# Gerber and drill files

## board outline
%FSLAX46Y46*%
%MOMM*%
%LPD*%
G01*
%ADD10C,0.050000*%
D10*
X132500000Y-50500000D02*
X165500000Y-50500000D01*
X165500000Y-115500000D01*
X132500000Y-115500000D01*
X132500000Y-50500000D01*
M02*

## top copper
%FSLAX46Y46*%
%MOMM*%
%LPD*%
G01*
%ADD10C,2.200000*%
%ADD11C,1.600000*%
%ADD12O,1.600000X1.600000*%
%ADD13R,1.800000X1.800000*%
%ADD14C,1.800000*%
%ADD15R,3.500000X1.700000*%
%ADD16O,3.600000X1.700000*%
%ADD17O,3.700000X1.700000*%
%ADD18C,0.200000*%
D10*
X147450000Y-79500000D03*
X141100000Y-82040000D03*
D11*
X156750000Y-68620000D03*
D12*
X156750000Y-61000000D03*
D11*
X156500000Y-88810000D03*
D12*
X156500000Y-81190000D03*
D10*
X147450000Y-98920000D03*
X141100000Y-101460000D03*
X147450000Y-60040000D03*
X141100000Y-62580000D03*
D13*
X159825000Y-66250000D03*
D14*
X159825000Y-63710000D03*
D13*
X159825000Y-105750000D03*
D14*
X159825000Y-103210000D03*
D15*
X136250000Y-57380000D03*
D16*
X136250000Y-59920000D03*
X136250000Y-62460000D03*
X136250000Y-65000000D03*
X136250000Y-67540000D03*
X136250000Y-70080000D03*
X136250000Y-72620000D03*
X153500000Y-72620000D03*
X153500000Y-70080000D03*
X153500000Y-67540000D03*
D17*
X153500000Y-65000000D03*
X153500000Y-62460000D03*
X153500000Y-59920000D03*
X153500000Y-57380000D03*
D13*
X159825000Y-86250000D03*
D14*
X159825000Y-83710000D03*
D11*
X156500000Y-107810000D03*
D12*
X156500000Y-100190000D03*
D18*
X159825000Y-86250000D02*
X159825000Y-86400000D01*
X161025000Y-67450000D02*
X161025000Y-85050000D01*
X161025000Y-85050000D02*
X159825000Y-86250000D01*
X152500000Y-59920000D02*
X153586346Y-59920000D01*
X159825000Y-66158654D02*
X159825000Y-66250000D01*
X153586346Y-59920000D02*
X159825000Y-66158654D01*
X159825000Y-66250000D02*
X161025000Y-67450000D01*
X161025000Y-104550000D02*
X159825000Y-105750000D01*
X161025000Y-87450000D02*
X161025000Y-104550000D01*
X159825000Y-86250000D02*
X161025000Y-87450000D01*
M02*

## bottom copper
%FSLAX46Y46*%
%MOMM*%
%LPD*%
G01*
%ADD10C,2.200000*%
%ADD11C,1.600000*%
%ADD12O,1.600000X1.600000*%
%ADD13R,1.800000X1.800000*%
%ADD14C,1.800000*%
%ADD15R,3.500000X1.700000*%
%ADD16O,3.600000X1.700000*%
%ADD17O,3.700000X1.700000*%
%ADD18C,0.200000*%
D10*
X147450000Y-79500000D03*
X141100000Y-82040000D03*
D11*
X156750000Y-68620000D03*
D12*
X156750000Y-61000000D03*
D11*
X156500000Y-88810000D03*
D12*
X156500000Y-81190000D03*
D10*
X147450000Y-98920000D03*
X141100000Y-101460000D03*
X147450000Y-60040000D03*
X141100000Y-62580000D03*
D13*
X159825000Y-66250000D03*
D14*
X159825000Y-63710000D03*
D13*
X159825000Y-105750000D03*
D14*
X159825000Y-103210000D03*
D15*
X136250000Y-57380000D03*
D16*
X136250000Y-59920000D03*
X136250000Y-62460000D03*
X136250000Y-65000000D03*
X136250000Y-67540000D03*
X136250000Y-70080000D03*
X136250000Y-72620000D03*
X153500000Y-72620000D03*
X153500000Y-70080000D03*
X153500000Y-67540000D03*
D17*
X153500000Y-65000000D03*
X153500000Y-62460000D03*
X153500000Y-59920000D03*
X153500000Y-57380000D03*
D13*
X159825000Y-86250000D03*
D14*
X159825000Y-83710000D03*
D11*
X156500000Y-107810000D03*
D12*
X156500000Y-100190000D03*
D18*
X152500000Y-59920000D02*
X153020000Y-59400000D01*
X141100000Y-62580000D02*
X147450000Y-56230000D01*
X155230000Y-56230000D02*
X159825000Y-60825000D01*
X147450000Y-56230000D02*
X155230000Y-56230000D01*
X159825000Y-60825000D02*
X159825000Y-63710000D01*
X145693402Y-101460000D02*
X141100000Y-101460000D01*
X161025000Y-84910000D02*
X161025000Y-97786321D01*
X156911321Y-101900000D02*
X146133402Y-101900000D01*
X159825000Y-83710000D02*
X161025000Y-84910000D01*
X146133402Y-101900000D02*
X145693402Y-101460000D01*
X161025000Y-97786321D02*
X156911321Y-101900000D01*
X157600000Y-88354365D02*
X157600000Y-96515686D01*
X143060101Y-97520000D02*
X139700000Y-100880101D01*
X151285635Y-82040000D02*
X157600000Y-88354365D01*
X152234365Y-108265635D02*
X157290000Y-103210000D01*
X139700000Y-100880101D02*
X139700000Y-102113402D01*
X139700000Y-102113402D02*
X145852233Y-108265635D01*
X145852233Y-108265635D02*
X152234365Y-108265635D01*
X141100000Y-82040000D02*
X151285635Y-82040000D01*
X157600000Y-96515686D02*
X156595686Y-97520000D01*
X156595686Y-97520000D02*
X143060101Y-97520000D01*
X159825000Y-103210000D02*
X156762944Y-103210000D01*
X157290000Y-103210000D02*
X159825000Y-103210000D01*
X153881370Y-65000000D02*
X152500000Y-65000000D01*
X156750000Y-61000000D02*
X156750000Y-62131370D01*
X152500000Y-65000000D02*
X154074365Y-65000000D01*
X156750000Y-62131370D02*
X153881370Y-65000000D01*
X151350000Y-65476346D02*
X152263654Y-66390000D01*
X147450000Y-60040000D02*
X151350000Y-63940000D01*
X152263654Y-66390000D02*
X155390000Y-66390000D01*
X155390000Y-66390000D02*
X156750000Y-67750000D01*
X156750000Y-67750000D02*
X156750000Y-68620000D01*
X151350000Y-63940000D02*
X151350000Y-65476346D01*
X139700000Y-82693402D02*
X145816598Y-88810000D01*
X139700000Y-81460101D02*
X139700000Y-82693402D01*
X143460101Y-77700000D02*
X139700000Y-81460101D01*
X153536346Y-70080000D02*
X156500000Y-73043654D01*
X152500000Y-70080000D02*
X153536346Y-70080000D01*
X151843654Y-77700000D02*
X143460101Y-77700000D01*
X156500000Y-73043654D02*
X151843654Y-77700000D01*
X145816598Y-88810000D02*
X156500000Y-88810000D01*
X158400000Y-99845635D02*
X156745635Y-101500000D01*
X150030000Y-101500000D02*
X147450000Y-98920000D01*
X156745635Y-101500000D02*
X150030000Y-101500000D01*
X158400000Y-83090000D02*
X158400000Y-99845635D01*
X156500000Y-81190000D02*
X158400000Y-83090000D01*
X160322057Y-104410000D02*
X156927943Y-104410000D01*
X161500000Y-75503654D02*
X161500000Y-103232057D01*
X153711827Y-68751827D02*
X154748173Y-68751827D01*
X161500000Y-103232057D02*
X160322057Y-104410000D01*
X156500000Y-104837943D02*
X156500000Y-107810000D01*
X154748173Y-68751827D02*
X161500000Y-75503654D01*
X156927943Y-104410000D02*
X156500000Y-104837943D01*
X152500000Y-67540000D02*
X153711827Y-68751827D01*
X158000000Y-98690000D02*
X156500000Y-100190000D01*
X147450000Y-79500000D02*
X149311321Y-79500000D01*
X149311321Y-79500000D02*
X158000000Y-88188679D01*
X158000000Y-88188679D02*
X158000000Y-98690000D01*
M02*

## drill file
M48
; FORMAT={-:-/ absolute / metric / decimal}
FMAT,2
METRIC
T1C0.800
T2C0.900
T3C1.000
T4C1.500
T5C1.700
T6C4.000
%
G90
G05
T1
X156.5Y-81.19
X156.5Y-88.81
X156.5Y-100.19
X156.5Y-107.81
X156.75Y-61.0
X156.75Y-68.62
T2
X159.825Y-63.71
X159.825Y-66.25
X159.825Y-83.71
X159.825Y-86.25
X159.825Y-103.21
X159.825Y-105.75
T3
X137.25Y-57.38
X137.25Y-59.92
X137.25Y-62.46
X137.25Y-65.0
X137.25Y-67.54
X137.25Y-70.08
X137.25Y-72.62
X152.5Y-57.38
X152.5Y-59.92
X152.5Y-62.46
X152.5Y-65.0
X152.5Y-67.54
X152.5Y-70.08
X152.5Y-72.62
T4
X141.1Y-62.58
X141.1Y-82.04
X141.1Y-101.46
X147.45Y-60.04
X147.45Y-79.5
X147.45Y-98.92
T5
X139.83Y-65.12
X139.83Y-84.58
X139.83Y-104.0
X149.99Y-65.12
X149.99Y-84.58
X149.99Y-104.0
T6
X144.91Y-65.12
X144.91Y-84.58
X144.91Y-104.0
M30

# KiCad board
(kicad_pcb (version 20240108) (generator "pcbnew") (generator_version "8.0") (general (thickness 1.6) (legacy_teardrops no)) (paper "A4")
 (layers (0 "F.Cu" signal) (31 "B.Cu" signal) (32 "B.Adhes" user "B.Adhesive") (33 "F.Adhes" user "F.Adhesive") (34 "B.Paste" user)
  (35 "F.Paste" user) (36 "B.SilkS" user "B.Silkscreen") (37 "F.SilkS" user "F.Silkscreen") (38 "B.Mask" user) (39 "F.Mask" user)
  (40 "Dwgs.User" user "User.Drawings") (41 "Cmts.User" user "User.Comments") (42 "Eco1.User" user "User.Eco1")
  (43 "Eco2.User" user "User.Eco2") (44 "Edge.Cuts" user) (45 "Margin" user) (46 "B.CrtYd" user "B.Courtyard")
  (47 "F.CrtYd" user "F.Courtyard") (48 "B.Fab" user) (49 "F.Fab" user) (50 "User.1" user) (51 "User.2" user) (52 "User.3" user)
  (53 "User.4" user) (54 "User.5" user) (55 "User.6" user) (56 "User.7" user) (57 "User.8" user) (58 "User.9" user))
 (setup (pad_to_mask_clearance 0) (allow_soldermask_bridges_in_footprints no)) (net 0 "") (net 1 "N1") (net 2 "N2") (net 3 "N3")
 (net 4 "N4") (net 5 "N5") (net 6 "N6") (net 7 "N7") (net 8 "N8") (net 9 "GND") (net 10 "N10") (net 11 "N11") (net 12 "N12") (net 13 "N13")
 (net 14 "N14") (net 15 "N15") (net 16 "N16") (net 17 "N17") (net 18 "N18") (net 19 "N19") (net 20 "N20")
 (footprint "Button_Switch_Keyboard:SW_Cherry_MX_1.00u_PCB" (layer "F.Cu") (at 147.45 79.5)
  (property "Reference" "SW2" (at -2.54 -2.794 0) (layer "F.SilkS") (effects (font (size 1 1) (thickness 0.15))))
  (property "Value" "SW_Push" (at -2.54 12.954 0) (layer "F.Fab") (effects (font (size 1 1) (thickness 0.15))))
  (pad "" np_thru_hole circle (at -7.62 5.08) (size 1.7 1.7) (drill 1.7) (layers "*.Cu" "*.Mask"))
  (pad "" np_thru_hole circle (at -2.54 5.08) (size 4 4) (drill 4) (layers "*.Cu" "*.Mask"))
  (pad "" np_thru_hole circle (at 2.54 5.08) (size 1.7 1.7) (drill 1.7) (layers "*.Cu" "*.Mask"))
  (pad "1" thru_hole circle (at 0 0) (size 2.2 2.2) (drill 1.5) (layers "*.Cu" "*.Mask") (remove_unused_layers no) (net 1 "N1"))
  (pad "2" thru_hole circle (at -6.35 2.54) (size 2.2 2.2) (drill 1.5) (layers "*.Cu" "*.Mask") (remove_unused_layers no) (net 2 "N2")))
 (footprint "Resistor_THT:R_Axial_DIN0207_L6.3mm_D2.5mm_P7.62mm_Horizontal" (layer "F.Cu") (at 156.75 68.62 90)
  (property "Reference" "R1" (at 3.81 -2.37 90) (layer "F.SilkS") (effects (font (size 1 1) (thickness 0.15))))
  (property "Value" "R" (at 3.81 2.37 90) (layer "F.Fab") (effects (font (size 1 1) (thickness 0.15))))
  (pad "1" thru_hole circle (at 0 0 90) (size 1.6 1.6) (drill 0.8) (layers "*.Cu" "*.Mask") (remove_unused_layers no) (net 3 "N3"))
  (pad "2" thru_hole oval (at 7.62 0 90) (size 1.6 1.6) (drill 0.8) (layers "*.Cu" "*.Mask") (remove_unused_layers no) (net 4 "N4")))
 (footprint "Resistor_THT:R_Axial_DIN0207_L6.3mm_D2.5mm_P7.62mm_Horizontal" (layer "F.Cu") (at 156.5 88.81 90)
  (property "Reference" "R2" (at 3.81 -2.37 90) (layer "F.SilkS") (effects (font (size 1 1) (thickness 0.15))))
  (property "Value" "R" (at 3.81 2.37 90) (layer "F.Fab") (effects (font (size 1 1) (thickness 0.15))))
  (pad "1" thru_hole circle (at 0 0 90) (size 1.6 1.6) (drill 0.8) (layers "*.Cu" "*.Mask") (remove_unused_layers no) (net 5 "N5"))
  (pad "2" thru_hole oval (at 7.62 0 90) (size 1.6 1.6) (drill 0.8) (layers "*.Cu" "*.Mask") (remove_unused_layers no) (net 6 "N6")))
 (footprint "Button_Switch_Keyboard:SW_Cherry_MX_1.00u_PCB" (layer "F.Cu") (at 147.45 98.92)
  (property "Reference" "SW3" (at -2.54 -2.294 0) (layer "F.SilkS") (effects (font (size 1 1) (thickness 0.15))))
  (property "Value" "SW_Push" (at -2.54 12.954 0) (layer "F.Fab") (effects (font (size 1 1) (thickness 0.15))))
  (pad "" np_thru_hole circle (at -7.62 5.08) (size 1.7 1.7) (drill 1.7) (layers "*.Cu" "*.Mask"))
  (pad "" np_thru_hole circle (at -2.54 5.08) (size 4 4) (drill 4) (layers "*.Cu" "*.Mask"))
  (pad "" np_thru_hole circle (at 2.54 5.08) (size 1.7 1.7) (drill 1.7) (layers "*.Cu" "*.Mask"))
  (pad "1" thru_hole circle (at 0 0) (size 2.2 2.2) (drill 1.5) (layers "*.Cu" "*.Mask") (remove_unused_layers no) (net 6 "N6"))
  (pad "2" thru_hole circle (at -6.35 2.54) (size 2.2 2.2) (drill 1.5) (layers "*.Cu" "*.Mask") (remove_unused_layers no) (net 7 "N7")))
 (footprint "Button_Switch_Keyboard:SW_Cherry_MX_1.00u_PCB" (layer "F.Cu") (at 147.45 60.04)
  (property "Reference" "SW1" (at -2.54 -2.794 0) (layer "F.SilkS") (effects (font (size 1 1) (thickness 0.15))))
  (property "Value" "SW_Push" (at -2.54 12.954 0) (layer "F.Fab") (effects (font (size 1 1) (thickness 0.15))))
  (pad "" np_thru_hole circle (at -7.62 5.08) (size 1.7 1.7) (drill 1.7) (layers "*.Cu" "*.Mask"))
  (pad "" np_thru_hole circle (at -2.54 5.08) (size 4 4) (drill 4) (layers "*.Cu" "*.Mask"))
  (pad "" np_thru_hole circle (at 2.54 5.08) (size 1.7 1.7) (drill 1.7) (layers "*.Cu" "*.Mask"))
  (pad "1" thru_hole circle (at 0 0) (size 2.2 2.2) (drill 1.5) (layers "*.Cu" "*.Mask") (remove_unused_layers no) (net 3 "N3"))
  (pad "2" thru_hole circle (at -6.35 2.54) (size 2.2 2.2) (drill 1.5) (layers "*.Cu" "*.Mask") (remove_unused_layers no) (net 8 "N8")))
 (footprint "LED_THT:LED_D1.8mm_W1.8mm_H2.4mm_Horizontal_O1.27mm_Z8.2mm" (layer "F.Cu") (at 159.825 66.25 90)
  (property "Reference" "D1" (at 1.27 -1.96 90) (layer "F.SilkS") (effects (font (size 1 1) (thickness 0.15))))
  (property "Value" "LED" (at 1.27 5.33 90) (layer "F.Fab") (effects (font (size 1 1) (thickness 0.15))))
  (pad "1" thru_hole rect (at 0 0 90) (size 1.8 1.8) (drill 0.9) (layers "*.Cu" "*.Mask") (remove_unused_layers no) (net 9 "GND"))
  (pad "2" thru_hole circle (at 2.54 0 90) (size 1.8 1.8) (drill 0.9) (layers "*.Cu" "*.Mask") (remove_unused_layers no) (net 8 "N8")))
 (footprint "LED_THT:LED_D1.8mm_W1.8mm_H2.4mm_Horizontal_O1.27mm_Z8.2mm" (layer "F.Cu") (at 159.825 105.75 90)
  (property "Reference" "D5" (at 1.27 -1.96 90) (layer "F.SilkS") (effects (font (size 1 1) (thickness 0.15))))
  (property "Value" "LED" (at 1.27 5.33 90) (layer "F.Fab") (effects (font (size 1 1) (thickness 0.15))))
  (pad "1" thru_hole rect (at 0 0 90) (size 1.8 1.8) (drill 0.9) (layers "*.Cu" "*.Mask") (remove_unused_layers no) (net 9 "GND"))
  (pad "2" thru_hole circle (at 2.54 0 90) (size 1.8 1.8) (drill 0.9) (layers "*.Cu" "*.Mask") (remove_unused_layers no) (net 2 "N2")))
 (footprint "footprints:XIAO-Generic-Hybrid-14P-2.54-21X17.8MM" (layer "F.Cu") (at 144.875 65)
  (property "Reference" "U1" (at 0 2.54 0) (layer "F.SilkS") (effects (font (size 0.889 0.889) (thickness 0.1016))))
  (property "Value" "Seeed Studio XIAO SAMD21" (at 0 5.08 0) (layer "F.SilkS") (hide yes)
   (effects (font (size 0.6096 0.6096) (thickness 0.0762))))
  (pad "1" thru_hole rect (at -7.625 -7.62) (size 3.5 1.7) (drill 1 (offset -1 0)) (layers "*.Cu" "*.Mask") (remove_unused_layers no)
   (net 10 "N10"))
  (pad "2" thru_hole oval (at -7.625 -5.08) (size 3.6 1.7) (drill 1 (offset -1 0)) (layers "*.Cu" "*.Mask") (remove_unused_layers no)
   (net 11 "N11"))
  (pad "3" thru_hole oval (at -7.625 -2.54) (size 3.6 1.7) (drill 1 (offset -1 0)) (layers "*.Cu" "*.Mask") (remove_unused_layers no)
   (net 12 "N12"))
  (pad "4" thru_hole oval (at -7.625 0) (size 3.6 1.7) (drill 1 (offset -1 0)) (layers "*.Cu" "*.Mask") (remove_unused_layers no)
   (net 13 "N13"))
  (pad "5" thru_hole oval (at -7.625 2.54) (size 3.6 1.7) (drill 1 (offset -1 0)) (layers "*.Cu" "*.Mask") (remove_unused_layers no)
   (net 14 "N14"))
  (pad "6" thru_hole oval (at -7.625 5.08 180) (size 3.6 1.7) (drill 1 (offset 1 0)) (layers "*.Cu" "*.Mask") (remove_unused_layers no)
   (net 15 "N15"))
  (pad "7" thru_hole oval (at -7.625 7.62) (size 3.6 1.7) (drill 1 (offset -1 0)) (layers "*.Cu" "*.Mask") (remove_unused_layers no)
   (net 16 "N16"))
  (pad "8" thru_hole oval (at 7.625 7.62) (size 3.6 1.7) (drill 1 (offset 1 0)) (layers "*.Cu" "*.Mask") (remove_unused_layers no)
   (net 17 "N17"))
  (pad "9" thru_hole oval (at 7.625 5.08) (size 3.6 1.7) (drill 1 (offset 1 0)) (layers "*.Cu" "*.Mask") (remove_unused_layers no)
   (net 5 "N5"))
  (pad "10" thru_hole oval (at 7.625 2.54) (size 3.6 1.7) (drill 1 (offset 1 0)) (layers "*.Cu" "*.Mask") (remove_unused_layers no)
   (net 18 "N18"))
  (pad "11" thru_hole oval (at 7.625 0) (size 3.7 1.7) (drill 1 (offset 1 0)) (layers "*.Cu" "*.Mask") (remove_unused_layers no)
   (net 4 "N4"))
  (pad "12" thru_hole oval (at 7.625 -2.54) (size 3.7 1.7) (drill 1 (offset 1 0)) (layers "*.Cu" "*.Mask") (remove_unused_layers no)
   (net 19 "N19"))
  (pad "13" thru_hole oval (at 7.625 -5.08) (size 3.7 1.7) (drill 1 (offset 1 0)) (layers "*.Cu" "*.Mask") (remove_unused_layers no)
   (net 9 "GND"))
  (pad "14" thru_hole oval (at 7.625 -7.62) (size 3.7 1.7) (drill 1 (offset 1 0)) (layers "*.Cu" "*.Mask") (remove_unused_layers no)
   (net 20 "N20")))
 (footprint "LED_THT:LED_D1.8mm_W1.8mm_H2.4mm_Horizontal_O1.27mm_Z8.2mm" (layer "F.Cu") (at 159.825 86.25 90)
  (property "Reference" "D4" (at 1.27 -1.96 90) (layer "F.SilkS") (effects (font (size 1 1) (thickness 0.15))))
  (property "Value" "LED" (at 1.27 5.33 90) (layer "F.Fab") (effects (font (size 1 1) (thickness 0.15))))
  (pad "1" thru_hole rect (at 0 0 90) (size 1.8 1.8) (drill 0.9) (layers "*.Cu" "*.Mask") (remove_unused_layers no) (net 9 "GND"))
  (pad "2" thru_hole circle (at 2.54 0 90) (size 1.8 1.8) (drill 0.9) (layers "*.Cu" "*.Mask") (remove_unused_layers no) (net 7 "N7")))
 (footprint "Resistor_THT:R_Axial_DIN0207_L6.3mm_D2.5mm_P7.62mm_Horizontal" (layer "F.Cu") (at 156.5 107.81 90)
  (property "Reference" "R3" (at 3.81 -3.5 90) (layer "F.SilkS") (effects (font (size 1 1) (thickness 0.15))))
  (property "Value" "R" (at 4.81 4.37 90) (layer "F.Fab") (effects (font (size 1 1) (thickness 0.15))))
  (pad "1" thru_hole circle (at 0 0 90) (size 1.6 1.6) (drill 0.8) (layers "*.Cu" "*.Mask") (remove_unused_layers no) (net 18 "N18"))
  (pad "2" thru_hole oval (at 7.62 0 90) (size 1.6 1.6) (drill 0.8) (layers "*.Cu" "*.Mask") (remove_unused_layers no) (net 1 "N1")))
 (gr_rect (start 132.5 50.5) (end 165.5 115.5) (stroke (width 0.05) (type default)) (fill none) (layer "Edge.Cuts"))
 (segment (start 159.825 86.25) (end 159.825 86.4) (width 0.2) (layer "F.Cu") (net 9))
 (segment (start 161.025 67.45) (end 161.025 85.05) (width 0.2) (layer "F.Cu") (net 9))
 (segment (start 161.025 85.05) (end 159.825 86.25) (width 0.2) (layer "F.Cu") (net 9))
 (segment (start 152.5 59.92) (end 153.586346 59.92) (width 0.2) (layer "F.Cu") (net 9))
 (segment (start 159.825 66.158654) (end 159.825 66.25) (width 0.2) (layer "F.Cu") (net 9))
 (segment (start 153.586346 59.92) (end 159.825 66.158654) (width 0.2) (layer "F.Cu") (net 9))
 (segment (start 159.825 66.25) (end 161.025 67.45) (width 0.2) (layer "F.Cu") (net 9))
 (segment (start 161.025 104.55) (end 159.825 105.75) (width 0.2) (layer "F.Cu") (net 9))
 (segment (start 161.025 87.45) (end 161.025 104.55) (width 0.2) (layer "F.Cu") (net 9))
 (segment (start 159.825 86.25) (end 161.025 87.45) (width 0.2) (layer "F.Cu") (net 9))
 (segment (start 152.5 59.92) (end 153.02 59.4) (width 0.2) (layer "B.Cu") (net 9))
 (segment (start 141.1 62.58) (end 147.45 56.23) (width 0.2) (layer "B.Cu") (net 8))
 (segment (start 155.23 56.23) (end 159.825 60.825) (width 0.2) (layer "B.Cu") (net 8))
 (segment (start 147.45 56.23) (end 155.23 56.23) (width 0.2) (layer "B.Cu") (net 8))
 (segment (start 159.825 60.825) (end 159.825 63.71) (width 0.2) (layer "B.Cu") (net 8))
 (segment (start 145.693402 101.46) (end 141.1 101.46) (width 0.2) (layer "B.Cu") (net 7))
 (segment (start 161.025 84.91) (end 161.025 97.786321) (width 0.2) (layer "B.Cu") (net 7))
 (segment (start 156.911321 101.9) (end 146.133402 101.9) (width 0.2) (layer "B.Cu") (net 7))
 (segment (start 159.825 83.71) (end 161.025 84.91) (width 0.2) (layer "B.Cu") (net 7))
 (segment (start 146.133402 101.9) (end 145.693402 101.46) (width 0.2) (layer "B.Cu") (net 7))
 (segment (start 161.025 97.786321) (end 156.911321 101.9) (width 0.2) (layer "B.Cu") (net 7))
 (segment (start 157.6 88.354365) (end 157.6 96.515686) (width 0.2) (layer "B.Cu") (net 2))
 (segment (start 143.060101 97.52) (end 139.7 100.880101) (width 0.2) (layer "B.Cu") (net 2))
 (segment (start 151.285635 82.04) (end 157.6 88.354365) (width 0.2) (layer "B.Cu") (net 2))
 (segment (start 152.234365 108.265635) (end 157.29 103.21) (width 0.2) (layer "B.Cu") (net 2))
 (segment (start 139.7 100.880101) (end 139.7 102.113402) (width 0.2) (layer "B.Cu") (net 2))
 (segment (start 139.7 102.113402) (end 145.852233 108.265635) (width 0.2) (layer "B.Cu") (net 2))
 (segment (start 145.852233 108.265635) (end 152.234365 108.265635) (width 0.2) (layer "B.Cu") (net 2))
 (segment (start 141.1 82.04) (end 151.285635 82.04) (width 0.2) (layer "B.Cu") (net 2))
 (segment (start 157.6 96.515686) (end 156.595686 97.52) (width 0.2) (layer "B.Cu") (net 2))
 (segment (start 156.595686 97.52) (end 143.060101 97.52) (width 0.2) (layer "B.Cu") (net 2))
 (segment (start 159.825 103.21) (end 156.762944 103.21) (width 0.2) (layer "B.Cu") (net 2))
 (segment (start 157.29 103.21) (end 159.825 103.21) (width 0.2) (layer "B.Cu") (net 2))
 (segment (start 153.88137 65) (end 152.5 65) (width 0.2) (layer "B.Cu") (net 4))
 (segment (start 156.75 61) (end 156.75 62.13137) (width 0.2) (layer "B.Cu") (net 4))
 (segment (start 152.5 65) (end 154.074365 65) (width 0.2) (layer "B.Cu") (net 4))
 (segment (start 156.75 62.13137) (end 153.88137 65) (width 0.2) (layer "B.Cu") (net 4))
 (segment (start 151.35 65.476346) (end 152.263654 66.39) (width 0.2) (layer "B.Cu") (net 3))
 (segment (start 147.45 60.04) (end 151.35 63.94) (width 0.2) (layer "B.Cu") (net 3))
 (segment (start 152.263654 66.39) (end 155.39 66.39) (width 0.2) (layer "B.Cu") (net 3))
 (segment (start 155.39 66.39) (end 156.75 67.75) (width 0.2) (layer "B.Cu") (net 3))
 (segment (start 156.75 67.75) (end 156.75 68.62) (width 0.2) (layer "B.Cu") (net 3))
 (segment (start 151.35 63.94) (end 151.35 65.476346) (width 0.2) (layer "B.Cu") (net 3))
 (segment (start 139.7 82.693402) (end 145.816598 88.81) (width 0.2) (layer "B.Cu") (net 5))
 (segment (start 139.7 81.460101) (end 139.7 82.693402) (width 0.2) (layer "B.Cu") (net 5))
 (segment (start 143.460101 77.7) (end 139.7 81.460101) (width 0.2) (layer "B.Cu") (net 5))
 (segment (start 153.536346 70.08) (end 156.5 73.043654) (width 0.2) (layer "B.Cu") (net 5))
 (segment (start 152.5 70.08) (end 153.536346 70.08) (width 0.2) (layer "B.Cu") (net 5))
 (segment (start 151.843654 77.7) (end 143.460101 77.7) (width 0.2) (layer "B.Cu") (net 5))
 (segment (start 156.5 73.043654) (end 151.843654 77.7) (width 0.2) (layer "B.Cu") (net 5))
 (segment (start 145.816598 88.81) (end 156.5 88.81) (width 0.2) (layer "B.Cu") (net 5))
 (segment (start 158.4 99.845635) (end 156.745635 101.5) (width 0.2) (layer "B.Cu") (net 6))
 (segment (start 150.03 101.5) (end 147.45 98.92) (width 0.2) (layer "B.Cu") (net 6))
 (segment (start 156.745635 101.5) (end 150.03 101.5) (width 0.2) (layer "B.Cu") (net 6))
 (segment (start 158.4 83.09) (end 158.4 99.845635) (width 0.2) (layer "B.Cu") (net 6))
 (segment (start 156.5 81.19) (end 158.4 83.09) (width 0.2) (layer "B.Cu") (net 6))
 (segment (start 160.322057 104.41) (end 156.927943 104.41) (width 0.2) (layer "B.Cu") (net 18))
 (segment (start 161.5 75.503654) (end 161.5 103.232057) (width 0.2) (layer "B.Cu") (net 18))
 (segment (start 153.711827 68.751827) (end 154.748173 68.751827) (width 0.2) (layer "B.Cu") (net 18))
 (segment (start 161.5 103.232057) (end 160.322057 104.41) (width 0.2) (layer "B.Cu") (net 18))
 (segment (start 156.5 104.837943) (end 156.5 107.81) (width 0.2) (layer "B.Cu") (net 18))
 (segment (start 154.748173 68.751827) (end 161.5 75.503654) (width 0.2) (layer "B.Cu") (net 18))
 (segment (start 156.927943 104.41) (end 156.5 104.837943) (width 0.2) (layer "B.Cu") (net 18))
 (segment (start 152.5 67.54) (end 153.711827 68.751827) (width 0.2) (layer "B.Cu") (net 18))
 (segment (start 158 98.69) (end 156.5 100.19) (width 0.2) (layer "B.Cu") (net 1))
 (segment (start 147.45 79.5) (end 149.311321 79.5) (width 0.2) (layer "B.Cu") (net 1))
 (segment (start 149.311321 79.5) (end 158 88.188679) (width 0.2) (layer "B.Cu") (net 1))
 (segment (start 158 88.188679) (end 158 98.69) (width 0.2) (layer "B.Cu") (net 1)))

